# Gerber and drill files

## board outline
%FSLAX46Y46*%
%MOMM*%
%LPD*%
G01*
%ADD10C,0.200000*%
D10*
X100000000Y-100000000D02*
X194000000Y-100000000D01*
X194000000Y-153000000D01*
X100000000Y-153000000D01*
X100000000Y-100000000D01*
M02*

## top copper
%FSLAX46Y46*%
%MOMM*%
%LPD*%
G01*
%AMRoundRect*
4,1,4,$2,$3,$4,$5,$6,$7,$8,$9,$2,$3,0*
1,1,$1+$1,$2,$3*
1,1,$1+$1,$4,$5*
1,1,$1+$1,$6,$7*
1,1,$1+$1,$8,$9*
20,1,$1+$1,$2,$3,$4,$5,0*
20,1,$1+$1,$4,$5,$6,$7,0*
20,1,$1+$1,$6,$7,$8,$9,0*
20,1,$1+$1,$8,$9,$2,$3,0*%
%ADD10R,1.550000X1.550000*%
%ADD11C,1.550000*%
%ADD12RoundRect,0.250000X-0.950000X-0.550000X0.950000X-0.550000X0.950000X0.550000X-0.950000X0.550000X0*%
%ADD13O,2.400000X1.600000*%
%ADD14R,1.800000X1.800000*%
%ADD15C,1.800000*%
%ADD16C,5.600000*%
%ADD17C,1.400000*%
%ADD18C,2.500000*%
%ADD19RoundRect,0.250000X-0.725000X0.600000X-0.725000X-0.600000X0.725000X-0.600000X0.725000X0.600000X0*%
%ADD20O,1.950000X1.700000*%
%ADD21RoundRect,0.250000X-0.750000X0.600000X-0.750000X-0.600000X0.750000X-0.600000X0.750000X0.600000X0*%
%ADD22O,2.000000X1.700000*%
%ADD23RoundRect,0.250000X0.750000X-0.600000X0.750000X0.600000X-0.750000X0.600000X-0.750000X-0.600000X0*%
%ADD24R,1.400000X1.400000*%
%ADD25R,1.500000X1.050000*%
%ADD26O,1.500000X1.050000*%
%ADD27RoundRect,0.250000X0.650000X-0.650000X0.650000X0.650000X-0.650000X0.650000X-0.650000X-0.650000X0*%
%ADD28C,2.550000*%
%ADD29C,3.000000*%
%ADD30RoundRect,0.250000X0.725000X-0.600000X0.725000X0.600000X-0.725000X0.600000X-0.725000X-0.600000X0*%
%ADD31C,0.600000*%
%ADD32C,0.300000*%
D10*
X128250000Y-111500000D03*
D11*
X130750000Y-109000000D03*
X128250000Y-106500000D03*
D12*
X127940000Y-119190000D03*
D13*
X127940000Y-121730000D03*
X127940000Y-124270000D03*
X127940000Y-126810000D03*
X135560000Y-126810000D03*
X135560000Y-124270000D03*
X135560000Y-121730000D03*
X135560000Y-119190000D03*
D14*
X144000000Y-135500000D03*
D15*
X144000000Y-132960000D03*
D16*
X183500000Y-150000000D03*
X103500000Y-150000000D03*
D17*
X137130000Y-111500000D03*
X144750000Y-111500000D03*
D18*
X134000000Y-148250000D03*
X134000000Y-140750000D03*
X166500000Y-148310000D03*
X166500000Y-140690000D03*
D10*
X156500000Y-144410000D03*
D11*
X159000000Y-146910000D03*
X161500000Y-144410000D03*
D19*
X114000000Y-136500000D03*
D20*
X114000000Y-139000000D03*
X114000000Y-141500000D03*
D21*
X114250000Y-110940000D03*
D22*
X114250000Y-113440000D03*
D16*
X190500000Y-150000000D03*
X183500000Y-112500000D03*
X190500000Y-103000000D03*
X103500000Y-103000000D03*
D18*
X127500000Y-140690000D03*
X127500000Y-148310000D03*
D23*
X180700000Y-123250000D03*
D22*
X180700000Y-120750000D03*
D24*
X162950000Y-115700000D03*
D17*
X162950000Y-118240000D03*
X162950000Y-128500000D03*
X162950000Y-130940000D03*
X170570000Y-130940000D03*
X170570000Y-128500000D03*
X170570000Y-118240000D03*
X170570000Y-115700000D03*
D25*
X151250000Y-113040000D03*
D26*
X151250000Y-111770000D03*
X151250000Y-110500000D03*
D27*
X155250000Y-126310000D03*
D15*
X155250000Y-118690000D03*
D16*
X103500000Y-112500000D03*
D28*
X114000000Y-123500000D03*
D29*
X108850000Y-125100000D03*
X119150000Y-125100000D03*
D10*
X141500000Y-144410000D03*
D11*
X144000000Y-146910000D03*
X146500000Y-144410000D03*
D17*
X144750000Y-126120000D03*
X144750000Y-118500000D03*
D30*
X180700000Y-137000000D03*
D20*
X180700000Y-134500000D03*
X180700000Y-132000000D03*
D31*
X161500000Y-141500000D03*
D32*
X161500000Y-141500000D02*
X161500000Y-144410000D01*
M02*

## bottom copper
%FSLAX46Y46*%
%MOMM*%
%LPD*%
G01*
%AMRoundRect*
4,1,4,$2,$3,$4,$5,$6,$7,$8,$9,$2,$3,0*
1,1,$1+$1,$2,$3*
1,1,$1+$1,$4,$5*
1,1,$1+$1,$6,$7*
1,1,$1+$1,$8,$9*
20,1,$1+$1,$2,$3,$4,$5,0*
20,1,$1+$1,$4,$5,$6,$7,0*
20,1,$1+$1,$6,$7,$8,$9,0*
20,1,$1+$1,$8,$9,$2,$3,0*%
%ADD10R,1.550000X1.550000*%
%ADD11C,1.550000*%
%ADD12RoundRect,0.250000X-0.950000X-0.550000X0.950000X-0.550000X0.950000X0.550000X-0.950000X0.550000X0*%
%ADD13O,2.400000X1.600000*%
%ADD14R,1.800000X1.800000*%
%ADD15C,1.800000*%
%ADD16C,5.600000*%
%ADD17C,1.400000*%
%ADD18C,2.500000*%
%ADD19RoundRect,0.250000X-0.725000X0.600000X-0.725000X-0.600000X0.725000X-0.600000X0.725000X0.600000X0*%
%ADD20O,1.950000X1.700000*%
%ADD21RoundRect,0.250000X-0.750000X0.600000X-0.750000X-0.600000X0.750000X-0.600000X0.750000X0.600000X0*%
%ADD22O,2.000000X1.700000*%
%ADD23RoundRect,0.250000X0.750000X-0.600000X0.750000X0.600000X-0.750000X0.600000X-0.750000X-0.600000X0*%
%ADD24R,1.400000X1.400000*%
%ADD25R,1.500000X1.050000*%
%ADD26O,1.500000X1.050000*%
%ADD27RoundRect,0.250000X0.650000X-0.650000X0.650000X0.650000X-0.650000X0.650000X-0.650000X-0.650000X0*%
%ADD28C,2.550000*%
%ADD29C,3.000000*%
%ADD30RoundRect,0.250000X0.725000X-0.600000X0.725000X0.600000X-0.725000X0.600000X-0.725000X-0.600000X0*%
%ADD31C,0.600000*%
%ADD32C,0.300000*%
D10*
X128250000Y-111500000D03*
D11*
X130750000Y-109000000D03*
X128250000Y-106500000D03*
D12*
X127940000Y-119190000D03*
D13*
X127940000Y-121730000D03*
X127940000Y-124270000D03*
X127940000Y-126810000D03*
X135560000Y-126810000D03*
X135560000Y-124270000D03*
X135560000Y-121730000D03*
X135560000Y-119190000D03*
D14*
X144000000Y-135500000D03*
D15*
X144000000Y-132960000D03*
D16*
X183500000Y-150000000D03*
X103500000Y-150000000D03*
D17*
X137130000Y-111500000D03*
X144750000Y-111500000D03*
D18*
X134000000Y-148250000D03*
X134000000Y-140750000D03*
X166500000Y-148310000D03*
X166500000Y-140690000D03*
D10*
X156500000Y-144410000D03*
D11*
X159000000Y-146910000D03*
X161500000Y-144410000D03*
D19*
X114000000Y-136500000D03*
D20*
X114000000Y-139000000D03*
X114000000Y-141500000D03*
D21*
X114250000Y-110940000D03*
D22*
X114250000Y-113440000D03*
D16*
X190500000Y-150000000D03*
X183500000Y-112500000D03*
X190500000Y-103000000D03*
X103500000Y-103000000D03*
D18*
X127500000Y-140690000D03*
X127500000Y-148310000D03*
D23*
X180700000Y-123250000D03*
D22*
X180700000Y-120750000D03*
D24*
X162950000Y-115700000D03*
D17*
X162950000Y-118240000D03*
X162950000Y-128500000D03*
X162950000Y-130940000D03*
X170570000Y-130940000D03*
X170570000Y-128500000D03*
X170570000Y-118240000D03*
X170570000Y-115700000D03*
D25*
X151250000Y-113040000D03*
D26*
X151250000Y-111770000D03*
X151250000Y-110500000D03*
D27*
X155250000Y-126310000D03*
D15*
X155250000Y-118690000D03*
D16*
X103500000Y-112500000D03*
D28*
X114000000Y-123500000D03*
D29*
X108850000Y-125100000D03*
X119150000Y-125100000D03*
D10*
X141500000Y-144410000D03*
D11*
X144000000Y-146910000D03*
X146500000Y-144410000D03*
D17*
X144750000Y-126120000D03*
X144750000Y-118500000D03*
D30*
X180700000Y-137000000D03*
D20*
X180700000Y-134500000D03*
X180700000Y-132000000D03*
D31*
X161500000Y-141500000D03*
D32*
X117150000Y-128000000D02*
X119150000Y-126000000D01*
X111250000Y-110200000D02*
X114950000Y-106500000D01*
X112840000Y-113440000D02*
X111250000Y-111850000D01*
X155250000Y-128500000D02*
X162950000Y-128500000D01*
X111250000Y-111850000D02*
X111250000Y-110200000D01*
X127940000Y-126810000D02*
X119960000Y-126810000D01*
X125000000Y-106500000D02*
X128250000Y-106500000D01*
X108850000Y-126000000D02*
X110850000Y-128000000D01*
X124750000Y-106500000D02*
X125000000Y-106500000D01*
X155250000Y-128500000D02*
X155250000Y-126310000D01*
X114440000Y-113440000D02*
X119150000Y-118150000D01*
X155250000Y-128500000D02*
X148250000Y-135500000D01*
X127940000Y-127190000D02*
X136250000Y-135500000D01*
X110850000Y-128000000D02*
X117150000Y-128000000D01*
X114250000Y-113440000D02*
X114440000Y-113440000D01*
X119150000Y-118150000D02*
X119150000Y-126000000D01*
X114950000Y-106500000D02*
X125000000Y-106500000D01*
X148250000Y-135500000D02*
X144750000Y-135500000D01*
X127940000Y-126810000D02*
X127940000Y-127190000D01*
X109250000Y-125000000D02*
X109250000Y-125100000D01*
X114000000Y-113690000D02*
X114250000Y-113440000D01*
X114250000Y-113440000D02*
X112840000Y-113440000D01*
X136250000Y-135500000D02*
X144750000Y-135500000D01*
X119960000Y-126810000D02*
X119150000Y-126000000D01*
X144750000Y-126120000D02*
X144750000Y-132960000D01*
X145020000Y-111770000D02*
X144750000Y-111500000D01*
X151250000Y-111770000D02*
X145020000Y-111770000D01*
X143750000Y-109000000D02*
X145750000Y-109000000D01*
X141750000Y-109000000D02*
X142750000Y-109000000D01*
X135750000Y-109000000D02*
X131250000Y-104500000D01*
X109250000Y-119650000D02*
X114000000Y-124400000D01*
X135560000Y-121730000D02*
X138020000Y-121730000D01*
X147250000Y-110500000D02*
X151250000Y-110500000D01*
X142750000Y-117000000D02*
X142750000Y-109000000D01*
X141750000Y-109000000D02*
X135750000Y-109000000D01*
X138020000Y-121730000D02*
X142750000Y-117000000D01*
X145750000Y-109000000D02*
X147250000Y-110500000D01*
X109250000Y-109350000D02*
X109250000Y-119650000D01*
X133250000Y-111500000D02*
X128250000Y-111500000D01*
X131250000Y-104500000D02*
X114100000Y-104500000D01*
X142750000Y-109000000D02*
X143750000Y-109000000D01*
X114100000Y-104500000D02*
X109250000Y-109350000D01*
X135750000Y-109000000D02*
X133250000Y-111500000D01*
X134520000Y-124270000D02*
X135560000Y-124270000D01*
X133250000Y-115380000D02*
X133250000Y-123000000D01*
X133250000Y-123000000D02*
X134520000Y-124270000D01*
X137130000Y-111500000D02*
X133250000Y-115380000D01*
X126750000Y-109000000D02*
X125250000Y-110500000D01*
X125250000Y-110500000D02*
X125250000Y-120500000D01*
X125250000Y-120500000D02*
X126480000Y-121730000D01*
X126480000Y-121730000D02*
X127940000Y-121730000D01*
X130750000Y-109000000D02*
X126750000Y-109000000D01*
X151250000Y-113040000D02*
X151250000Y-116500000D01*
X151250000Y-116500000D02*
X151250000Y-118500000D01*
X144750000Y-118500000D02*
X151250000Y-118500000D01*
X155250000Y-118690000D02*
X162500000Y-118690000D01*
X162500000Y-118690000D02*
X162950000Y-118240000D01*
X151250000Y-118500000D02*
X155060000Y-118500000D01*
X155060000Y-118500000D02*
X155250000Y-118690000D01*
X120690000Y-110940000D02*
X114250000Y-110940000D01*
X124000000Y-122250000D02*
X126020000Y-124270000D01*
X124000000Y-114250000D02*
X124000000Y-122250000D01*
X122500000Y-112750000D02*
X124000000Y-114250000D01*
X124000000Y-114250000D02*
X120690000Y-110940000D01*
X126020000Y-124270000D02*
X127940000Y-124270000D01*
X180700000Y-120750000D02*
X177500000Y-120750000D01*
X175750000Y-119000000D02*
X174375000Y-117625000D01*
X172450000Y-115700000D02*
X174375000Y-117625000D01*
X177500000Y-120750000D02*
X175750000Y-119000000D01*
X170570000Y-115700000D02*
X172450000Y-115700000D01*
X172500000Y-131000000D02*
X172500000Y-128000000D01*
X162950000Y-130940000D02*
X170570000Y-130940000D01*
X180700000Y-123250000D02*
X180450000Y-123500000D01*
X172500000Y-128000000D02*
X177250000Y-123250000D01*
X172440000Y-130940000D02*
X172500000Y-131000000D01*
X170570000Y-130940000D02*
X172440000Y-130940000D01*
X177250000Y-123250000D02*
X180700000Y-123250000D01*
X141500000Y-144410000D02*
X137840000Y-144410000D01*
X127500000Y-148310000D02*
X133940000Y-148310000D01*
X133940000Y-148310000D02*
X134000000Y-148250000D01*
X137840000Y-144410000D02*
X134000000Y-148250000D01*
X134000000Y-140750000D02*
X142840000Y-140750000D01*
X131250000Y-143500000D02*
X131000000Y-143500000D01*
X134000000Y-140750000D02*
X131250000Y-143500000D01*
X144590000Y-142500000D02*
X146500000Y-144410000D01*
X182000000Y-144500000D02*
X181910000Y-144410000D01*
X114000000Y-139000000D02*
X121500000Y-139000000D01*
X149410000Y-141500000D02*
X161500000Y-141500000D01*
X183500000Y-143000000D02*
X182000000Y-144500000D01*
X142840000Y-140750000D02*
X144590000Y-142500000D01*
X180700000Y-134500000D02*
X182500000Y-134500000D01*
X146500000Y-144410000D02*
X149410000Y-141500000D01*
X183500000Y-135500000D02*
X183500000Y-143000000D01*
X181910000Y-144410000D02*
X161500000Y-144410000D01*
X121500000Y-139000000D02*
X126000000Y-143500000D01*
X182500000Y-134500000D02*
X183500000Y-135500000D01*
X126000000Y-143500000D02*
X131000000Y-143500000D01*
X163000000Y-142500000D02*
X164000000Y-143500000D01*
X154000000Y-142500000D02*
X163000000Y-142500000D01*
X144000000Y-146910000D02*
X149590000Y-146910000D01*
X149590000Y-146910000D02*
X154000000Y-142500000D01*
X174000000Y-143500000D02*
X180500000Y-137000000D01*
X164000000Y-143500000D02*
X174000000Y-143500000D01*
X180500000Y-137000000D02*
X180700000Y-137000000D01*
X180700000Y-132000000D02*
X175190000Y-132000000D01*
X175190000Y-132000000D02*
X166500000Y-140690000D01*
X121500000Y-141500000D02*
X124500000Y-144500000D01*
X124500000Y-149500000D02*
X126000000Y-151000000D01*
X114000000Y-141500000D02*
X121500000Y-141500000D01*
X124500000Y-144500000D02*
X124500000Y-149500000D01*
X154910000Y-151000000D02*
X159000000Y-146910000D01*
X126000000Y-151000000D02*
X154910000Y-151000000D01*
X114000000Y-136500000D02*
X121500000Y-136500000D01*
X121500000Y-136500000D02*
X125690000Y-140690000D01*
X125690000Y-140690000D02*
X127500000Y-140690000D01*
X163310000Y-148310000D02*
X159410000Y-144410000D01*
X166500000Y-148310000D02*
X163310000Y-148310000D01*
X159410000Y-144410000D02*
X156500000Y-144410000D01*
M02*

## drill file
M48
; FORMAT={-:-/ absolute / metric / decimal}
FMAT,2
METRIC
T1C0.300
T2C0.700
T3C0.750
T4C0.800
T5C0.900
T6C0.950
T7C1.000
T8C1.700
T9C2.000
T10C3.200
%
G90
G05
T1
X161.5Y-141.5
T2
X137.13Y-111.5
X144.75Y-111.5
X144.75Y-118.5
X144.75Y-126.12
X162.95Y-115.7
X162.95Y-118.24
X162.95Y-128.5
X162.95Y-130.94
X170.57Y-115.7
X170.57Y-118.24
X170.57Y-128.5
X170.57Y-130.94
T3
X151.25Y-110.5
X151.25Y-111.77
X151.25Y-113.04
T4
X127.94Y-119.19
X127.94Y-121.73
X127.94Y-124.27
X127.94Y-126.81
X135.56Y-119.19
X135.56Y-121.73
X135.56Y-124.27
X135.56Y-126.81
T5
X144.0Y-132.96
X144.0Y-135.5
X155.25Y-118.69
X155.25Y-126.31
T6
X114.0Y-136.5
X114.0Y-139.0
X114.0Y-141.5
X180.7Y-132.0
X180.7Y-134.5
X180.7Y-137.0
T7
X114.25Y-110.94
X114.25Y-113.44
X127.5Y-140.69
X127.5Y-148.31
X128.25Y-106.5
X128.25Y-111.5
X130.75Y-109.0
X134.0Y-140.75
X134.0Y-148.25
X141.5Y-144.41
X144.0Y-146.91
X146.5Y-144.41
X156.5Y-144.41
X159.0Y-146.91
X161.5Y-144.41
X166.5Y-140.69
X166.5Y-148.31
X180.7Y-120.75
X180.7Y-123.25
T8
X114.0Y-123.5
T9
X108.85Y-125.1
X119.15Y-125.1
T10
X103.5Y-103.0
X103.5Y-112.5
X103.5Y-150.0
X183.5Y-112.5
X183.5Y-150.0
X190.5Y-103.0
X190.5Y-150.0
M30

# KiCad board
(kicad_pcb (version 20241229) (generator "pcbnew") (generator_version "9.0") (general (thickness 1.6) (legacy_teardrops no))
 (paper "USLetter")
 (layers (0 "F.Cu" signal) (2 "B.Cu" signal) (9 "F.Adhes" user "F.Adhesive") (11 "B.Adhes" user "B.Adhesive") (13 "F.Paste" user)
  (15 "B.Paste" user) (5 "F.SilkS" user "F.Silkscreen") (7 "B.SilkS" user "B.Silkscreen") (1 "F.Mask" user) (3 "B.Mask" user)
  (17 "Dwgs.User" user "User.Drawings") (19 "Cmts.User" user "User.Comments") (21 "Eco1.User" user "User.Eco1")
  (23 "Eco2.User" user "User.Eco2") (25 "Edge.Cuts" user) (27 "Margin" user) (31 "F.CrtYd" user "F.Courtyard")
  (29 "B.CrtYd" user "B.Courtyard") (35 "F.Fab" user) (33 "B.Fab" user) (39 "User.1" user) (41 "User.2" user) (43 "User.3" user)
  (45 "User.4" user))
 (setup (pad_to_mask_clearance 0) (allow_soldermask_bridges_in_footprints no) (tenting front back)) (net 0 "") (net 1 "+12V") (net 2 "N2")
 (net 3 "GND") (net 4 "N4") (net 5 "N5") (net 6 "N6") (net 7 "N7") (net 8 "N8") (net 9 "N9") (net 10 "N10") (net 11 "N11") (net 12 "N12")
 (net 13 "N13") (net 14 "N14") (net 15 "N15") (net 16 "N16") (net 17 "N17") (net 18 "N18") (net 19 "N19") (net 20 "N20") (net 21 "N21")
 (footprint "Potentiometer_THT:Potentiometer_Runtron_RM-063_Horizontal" (layer "F.Cu") (at 128.25 111.5 90)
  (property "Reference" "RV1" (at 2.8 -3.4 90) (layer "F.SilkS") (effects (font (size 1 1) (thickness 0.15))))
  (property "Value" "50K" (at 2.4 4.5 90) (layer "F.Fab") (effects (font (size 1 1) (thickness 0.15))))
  (pad "1" thru_hole rect (at 0 0 90) (size 1.55 1.55) (drill 1) (layers "*.Cu" "*.Mask") (remove_unused_layers no) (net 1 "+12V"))
  (pad "2" thru_hole circle (at 2.5 2.5 90) (size 1.55 1.55) (drill 1) (layers "*.Cu" "*.Mask") (remove_unused_layers no) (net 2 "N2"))
  (pad "3" thru_hole circle (at 5 0 90) (size 1.55 1.55) (drill 1) (layers "*.Cu" "*.Mask") (remove_unused_layers no) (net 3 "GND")))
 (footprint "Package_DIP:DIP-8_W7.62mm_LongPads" (layer "F.Cu") (at 127.94 119.19)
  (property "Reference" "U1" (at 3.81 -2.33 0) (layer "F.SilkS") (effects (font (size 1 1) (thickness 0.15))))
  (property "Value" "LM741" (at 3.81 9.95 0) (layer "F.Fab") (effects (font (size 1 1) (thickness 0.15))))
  (pad "1" thru_hole roundrect (at 0 0) (size 2.4 1.6) (drill 0.8) (layers "*.Cu" "*.Mask") (remove_unused_layers no)
   (roundrect_rratio 0.15625) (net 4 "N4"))
  (pad "2" thru_hole oval (at 0 2.54) (size 2.4 1.6) (drill 0.8) (layers "*.Cu" "*.Mask") (remove_unused_layers no) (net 2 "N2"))
  (pad "3" thru_hole oval (at 0 5.08) (size 2.4 1.6) (drill 0.8) (layers "*.Cu" "*.Mask") (remove_unused_layers no) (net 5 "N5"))
  (pad "4" thru_hole oval (at 0 7.62) (size 2.4 1.6) (drill 0.8) (layers "*.Cu" "*.Mask") (remove_unused_layers no) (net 3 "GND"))
  (pad "5" thru_hole oval (at 7.62 7.62) (size 2.4 1.6) (drill 0.8) (layers "*.Cu" "*.Mask") (remove_unused_layers no) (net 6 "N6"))
  (pad "6" thru_hole oval (at 7.62 5.08) (size 2.4 1.6) (drill 0.8) (layers "*.Cu" "*.Mask") (remove_unused_layers no) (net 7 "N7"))
  (pad "7" thru_hole oval (at 7.62 2.54) (size 2.4 1.6) (drill 0.8) (layers "*.Cu" "*.Mask") (remove_unused_layers no) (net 1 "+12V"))
  (pad "8" thru_hole oval (at 7.62 0) (size 2.4 1.6) (drill 0.8) (layers "*.Cu" "*.Mask") (remove_unused_layers no) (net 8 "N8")))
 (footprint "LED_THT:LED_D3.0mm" (layer "F.Cu") (at 144 135.5 90)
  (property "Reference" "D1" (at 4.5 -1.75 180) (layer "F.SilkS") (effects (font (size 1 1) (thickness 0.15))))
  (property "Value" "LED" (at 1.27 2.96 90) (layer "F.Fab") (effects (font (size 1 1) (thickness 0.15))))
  (pad "1" thru_hole rect (at 0 0 90) (size 1.8 1.8) (drill 0.9) (layers "*.Cu" "*.Mask") (remove_unused_layers no) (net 3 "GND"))
  (pad "2" thru_hole circle (at 2.54 0 90) (size 1.8 1.8) (drill 0.9) (layers "*.Cu" "*.Mask") (remove_unused_layers no) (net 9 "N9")))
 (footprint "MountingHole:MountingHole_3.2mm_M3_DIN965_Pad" (layer "F.Cu") (at 183.5 150)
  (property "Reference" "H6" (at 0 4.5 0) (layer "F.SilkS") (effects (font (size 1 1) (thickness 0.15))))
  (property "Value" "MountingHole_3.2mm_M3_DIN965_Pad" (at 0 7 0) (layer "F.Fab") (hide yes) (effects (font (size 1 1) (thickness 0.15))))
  (pad "1" thru_hole circle (at 0 0) (size 5.6 5.6) (drill 3.2) (layers "*.Cu" "*.Mask") (remove_unused_layers no) (zone_connect 2)))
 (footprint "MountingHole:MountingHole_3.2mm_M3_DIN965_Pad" (layer "F.Cu") (at 103.5 150)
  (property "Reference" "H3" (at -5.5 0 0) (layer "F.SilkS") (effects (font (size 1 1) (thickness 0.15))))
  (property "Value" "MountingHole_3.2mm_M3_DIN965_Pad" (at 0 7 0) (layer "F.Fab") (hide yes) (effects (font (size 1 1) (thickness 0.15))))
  (pad "1" thru_hole circle (at 0 0) (size 5.6 5.6) (drill 3.2) (layers "*.Cu" "*.Mask") (remove_unused_layers no) (zone_connect 2)))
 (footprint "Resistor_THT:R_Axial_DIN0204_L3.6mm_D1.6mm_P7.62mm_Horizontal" (layer "F.Cu") (at 137.13 111.5)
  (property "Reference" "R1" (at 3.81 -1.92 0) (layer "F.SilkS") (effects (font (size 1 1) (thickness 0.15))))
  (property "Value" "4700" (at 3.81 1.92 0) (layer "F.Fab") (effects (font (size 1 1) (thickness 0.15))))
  (pad "1" thru_hole circle (at 0 0) (size 1.4 1.4) (drill 0.7) (layers "*.Cu" "*.Mask") (remove_unused_layers no) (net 7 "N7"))
  (pad "2" thru_hole circle (at 7.62 0) (size 1.4 1.4) (drill 0.7) (layers "*.Cu" "*.Mask") (remove_unused_layers no) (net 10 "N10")))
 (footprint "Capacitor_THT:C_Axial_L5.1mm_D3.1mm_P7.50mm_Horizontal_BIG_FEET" (layer "F.Cu") (at 134 148.25 90)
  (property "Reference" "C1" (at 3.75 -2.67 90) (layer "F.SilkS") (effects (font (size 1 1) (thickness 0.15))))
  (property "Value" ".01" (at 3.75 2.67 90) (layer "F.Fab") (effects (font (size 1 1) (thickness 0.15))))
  (pad "1" thru_hole circle (at 0 0 90) (size 2.5 2.5) (drill 1) (layers "*.Cu" "*.Mask") (remove_unused_layers no) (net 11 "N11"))
  (pad "2" thru_hole circle (at 7.5 0 90) (size 2.5 2.5) (drill 1) (layers "*.Cu" "*.Mask") (remove_unused_layers no) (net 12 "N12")))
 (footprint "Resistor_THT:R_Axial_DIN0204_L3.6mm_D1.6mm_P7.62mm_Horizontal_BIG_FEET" (layer "F.Cu") (at 166.5 148.31 90)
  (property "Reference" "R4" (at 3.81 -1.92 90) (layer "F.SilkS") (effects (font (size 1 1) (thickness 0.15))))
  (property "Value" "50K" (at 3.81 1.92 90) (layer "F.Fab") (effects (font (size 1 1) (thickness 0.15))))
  (pad "1" thru_hole circle (at 0 0 90) (size 2.5 2.5) (drill 1) (layers "*.Cu" "*.Mask") (remove_unused_layers no) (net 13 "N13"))
  (pad "2" thru_hole circle (at 7.62 0 90) (size 2.5 2.5) (drill 1) (layers "*.Cu" "*.Mask") (remove_unused_layers no) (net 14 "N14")))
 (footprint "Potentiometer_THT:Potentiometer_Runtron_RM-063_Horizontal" (layer "F.Cu") (at 156.5 144.41)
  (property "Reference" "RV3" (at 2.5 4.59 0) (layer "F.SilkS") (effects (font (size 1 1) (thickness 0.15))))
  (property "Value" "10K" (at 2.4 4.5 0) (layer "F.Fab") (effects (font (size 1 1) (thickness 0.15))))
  (pad "1" thru_hole rect (at 0 0) (size 1.55 1.55) (drill 1) (layers "*.Cu" "*.Mask") (remove_unused_layers no) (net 13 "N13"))
  (pad "2" thru_hole circle (at 2.5 2.5) (size 1.55 1.55) (drill 1) (layers "*.Cu" "*.Mask") (remove_unused_layers no) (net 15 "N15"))
  (pad "3" thru_hole circle (at 5 0) (size 1.55 1.55) (drill 1) (layers "*.Cu" "*.Mask") (remove_unused_layers no) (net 12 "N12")))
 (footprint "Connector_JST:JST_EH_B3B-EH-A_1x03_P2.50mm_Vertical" (layer "F.Cu") (at 114 136.5 -90)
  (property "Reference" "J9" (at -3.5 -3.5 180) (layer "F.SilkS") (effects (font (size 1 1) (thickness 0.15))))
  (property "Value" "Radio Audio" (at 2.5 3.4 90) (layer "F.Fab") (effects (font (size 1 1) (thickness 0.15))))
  (pad "1" thru_hole roundrect (at 0 0 270) (size 1.7 1.95) (drill 0.95) (layers "*.Cu" "*.Mask") (remove_unused_layers no)
   (roundrect_rratio 0.147059) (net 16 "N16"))
  (pad "2" thru_hole oval (at 2.5 0 270) (size 1.7 1.95) (drill 0.95) (layers "*.Cu" "*.Mask") (remove_unused_layers no) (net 12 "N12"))
  (pad "3" thru_hole oval (at 5 0 270) (size 1.7 1.95) (drill 0.95) (layers "*.Cu" "*.Mask") (remove_unused_layers no) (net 15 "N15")))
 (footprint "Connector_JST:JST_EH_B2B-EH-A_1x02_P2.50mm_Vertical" (layer "F.Cu") (at 114.25 110.94 -90)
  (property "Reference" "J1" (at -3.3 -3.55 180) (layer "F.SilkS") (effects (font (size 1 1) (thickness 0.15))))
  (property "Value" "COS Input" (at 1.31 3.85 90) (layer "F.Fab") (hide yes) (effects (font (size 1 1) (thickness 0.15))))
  (pad "1" thru_hole roundrect (at 0 0 270) (size 1.7 2) (drill 1) (layers "*.Cu" "*.Mask") (remove_unused_layers no)
   (roundrect_rratio 0.147059) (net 5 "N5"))
  (pad "2" thru_hole oval (at 2.5 0 270) (size 1.7 2) (drill 1) (layers "*.Cu" "*.Mask") (remove_unused_layers no) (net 3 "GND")))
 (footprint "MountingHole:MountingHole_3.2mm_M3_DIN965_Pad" (layer "F.Cu") (at 190.5 150)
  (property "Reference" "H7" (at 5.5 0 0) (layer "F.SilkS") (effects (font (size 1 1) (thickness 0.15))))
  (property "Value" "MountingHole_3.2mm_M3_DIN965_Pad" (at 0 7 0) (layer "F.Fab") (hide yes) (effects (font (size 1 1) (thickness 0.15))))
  (pad "1" thru_hole circle (at 0 0) (size 5.6 5.6) (drill 3.2) (layers "*.Cu" "*.Mask") (remove_unused_layers no) (zone_connect 2)))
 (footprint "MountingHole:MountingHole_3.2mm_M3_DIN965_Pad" (layer "F.Cu") (at 183.5 112.5)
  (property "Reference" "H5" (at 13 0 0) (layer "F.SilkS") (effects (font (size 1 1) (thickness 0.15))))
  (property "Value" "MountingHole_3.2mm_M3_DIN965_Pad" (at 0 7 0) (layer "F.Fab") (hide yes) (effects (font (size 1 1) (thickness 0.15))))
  (pad "1" thru_hole circle (at 0 0) (size 5.6 5.6) (drill 3.2) (layers "*.Cu" "*.Mask") (remove_unused_layers no) (zone_connect 2)))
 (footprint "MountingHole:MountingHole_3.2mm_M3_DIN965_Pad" (layer "F.Cu") (at 190.5 103)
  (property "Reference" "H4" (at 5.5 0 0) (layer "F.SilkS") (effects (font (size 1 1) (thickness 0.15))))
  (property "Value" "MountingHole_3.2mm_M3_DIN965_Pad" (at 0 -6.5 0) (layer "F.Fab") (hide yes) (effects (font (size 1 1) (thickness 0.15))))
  (pad "1" thru_hole circle (at 0 0) (size 5.6 5.6) (drill 3.2) (layers "*.Cu" "*.Mask") (remove_unused_layers no) (zone_connect 2)))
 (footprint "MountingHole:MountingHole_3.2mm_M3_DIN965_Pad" (layer "F.Cu") (at 103.5 103)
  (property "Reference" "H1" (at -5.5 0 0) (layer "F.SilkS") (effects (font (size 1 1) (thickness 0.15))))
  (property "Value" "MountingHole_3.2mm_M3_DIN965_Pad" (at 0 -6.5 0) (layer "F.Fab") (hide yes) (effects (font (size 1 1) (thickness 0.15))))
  (pad "1" thru_hole circle (at 0 0) (size 5.6 5.6) (drill 3.2) (layers "*.Cu" "*.Mask") (remove_unused_layers no) (zone_connect 2)))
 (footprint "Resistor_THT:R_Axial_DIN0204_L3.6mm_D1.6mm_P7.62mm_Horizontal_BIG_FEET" (layer "F.Cu") (at 127.5 140.69 -90)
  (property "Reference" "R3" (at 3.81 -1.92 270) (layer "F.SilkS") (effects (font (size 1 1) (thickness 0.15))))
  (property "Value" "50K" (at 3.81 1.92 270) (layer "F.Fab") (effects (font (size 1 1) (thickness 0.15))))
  (pad "1" thru_hole circle (at 0 0 270) (size 2.5 2.5) (drill 1) (layers "*.Cu" "*.Mask") (remove_unused_layers no) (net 16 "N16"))
  (pad "2" thru_hole circle (at 7.62 0 270) (size 2.5 2.5) (drill 1) (layers "*.Cu" "*.Mask") (remove_unused_layers no) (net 11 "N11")))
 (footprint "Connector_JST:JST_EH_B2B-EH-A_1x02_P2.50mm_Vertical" (layer "F.Cu") (at 180.7 123.25 90)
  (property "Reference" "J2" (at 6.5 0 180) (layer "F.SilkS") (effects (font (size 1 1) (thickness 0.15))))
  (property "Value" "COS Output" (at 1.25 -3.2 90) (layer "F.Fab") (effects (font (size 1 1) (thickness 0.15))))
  (pad "1" thru_hole roundrect (at 0 0 90) (size 1.7 2) (drill 1) (layers "*.Cu" "*.Mask") (remove_unused_layers no)
   (roundrect_rratio 0.147059) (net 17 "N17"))
  (pad "2" thru_hole oval (at 2.5 0 90) (size 1.7 2) (drill 1) (layers "*.Cu" "*.Mask") (remove_unused_layers no) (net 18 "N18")))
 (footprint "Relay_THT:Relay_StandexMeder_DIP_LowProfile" (layer "F.Cu") (at 162.95 115.7)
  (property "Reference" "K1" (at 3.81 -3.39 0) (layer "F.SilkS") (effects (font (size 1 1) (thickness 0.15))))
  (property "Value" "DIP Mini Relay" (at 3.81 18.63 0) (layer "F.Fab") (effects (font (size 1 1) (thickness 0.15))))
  (pad "1" thru_hole rect (at 0 0) (size 1.4 1.4) (drill 0.7) (layers "*.Cu" "*.Mask") (remove_unused_layers no) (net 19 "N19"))
  (pad "2" thru_hole circle (at 0 2.54) (size 1.4 1.4) (drill 0.7) (layers "*.Cu" "*.Mask") (remove_unused_layers no) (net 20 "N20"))
  (pad "6" thru_hole circle (at 0 12.8) (size 1.4 1.4) (drill 0.7) (layers "*.Cu" "*.Mask") (remove_unused_layers no) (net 3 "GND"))
  (pad "7" thru_hole circle (at 0 15.24) (size 1.4 1.4) (drill 0.7) (layers "*.Cu" "*.Mask") (remove_unused_layers no) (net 17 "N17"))
  (pad "8" thru_hole circle (at 7.62 15.24) (size 1.4 1.4) (drill 0.7) (layers "*.Cu" "*.Mask") (remove_unused_layers no) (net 17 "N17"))
  (pad "9" thru_hole circle (at 7.62 12.8) (size 1.4 1.4) (drill 0.7) (layers "*.Cu" "*.Mask") (remove_unused_layers no))
  (pad "13" thru_hole circle (at 7.62 2.54) (size 1.4 1.4) (drill 0.7) (layers "*.Cu" "*.Mask") (remove_unused_layers no))
  (pad "14" thru_hole circle (at 7.62 0) (size 1.4 1.4) (drill 0.7) (layers "*.Cu" "*.Mask") (remove_unused_layers no) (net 18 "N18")))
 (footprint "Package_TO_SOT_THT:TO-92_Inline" (layer "F.Cu") (at 151.25 113.04 90)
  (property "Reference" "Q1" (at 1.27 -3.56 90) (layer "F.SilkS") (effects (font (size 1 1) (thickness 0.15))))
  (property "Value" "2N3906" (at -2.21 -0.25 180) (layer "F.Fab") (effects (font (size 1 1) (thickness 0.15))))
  (pad "1" thru_hole rect (at 0 0 90) (size 1.05 1.5) (drill 0.75) (layers "*.Cu" "*.Mask") (remove_unused_layers no) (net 20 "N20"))
  (pad "2" thru_hole oval (at 1.27 0 90) (size 1.05 1.5) (drill 0.75) (layers "*.Cu" "*.Mask") (remove_unused_layers no) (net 10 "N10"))
  (pad "3" thru_hole oval (at 2.54 0 90) (size 1.05 1.5) (drill 0.75) (layers "*.Cu" "*.Mask") (remove_unused_layers no) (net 1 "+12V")))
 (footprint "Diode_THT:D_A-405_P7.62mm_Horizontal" (layer "F.Cu") (at 155.25 126.31 90)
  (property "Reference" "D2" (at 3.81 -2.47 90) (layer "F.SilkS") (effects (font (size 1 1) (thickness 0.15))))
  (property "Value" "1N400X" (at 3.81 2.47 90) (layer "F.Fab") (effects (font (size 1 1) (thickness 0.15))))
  (pad "1" thru_hole roundrect (at 0 0 90) (size 1.8 1.8) (drill 0.9) (layers "*.Cu" "*.Mask") (remove_unused_layers no)
   (roundrect_rratio 0.138889) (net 3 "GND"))
  (pad "2" thru_hole circle (at 7.62 0 90) (size 1.8 1.8) (drill 0.9) (layers "*.Cu" "*.Mask") (remove_unused_layers no) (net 20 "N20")))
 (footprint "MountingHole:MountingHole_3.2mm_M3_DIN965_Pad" (layer "F.Cu") (at 103.5 112.5)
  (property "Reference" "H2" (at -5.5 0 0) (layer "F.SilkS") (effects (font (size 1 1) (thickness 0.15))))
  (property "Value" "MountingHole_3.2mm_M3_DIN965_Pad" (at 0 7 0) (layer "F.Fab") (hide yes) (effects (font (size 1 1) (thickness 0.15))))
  (pad "1" thru_hole circle (at 0 0) (size 5.6 5.6) (drill 3.2) (layers "*.Cu" "*.Mask") (remove_unused_layers no) (zone_connect 2)))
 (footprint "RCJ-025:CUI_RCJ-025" (layer "F.Cu") (at 114 125.1)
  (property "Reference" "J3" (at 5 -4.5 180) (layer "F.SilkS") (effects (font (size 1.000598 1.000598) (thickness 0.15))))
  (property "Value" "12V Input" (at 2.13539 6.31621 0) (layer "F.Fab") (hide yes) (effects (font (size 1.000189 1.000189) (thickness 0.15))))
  (pad "1" thru_hole circle (at 0 -1.6) (size 2.55 2.55) (drill 1.7) (layers "*.Cu" "*.Mask") (remove_unused_layers no) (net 1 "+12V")
   (solder_mask_margin 0.102))
  (pad "2" thru_hole circle (at -5.15 0) (size 3 3) (drill 2) (layers "*.Cu" "*.Mask") (remove_unused_layers no) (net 3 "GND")
   (solder_mask_margin 0.102))
  (pad "2" thru_hole circle (at 5.15 0) (size 3 3) (drill 2) (layers "*.Cu" "*.Mask") (remove_unused_layers no) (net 3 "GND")
   (solder_mask_margin 0.102)))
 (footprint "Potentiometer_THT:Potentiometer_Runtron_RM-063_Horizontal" (layer "F.Cu") (at 141.5 144.41)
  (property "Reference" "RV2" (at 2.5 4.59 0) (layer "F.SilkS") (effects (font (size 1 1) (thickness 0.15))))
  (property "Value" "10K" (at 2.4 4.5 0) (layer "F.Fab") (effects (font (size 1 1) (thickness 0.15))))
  (pad "1" thru_hole rect (at 0 0) (size 1.55 1.55) (drill 1) (layers "*.Cu" "*.Mask") (remove_unused_layers no) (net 11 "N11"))
  (pad "2" thru_hole circle (at 2.5 2.5) (size 1.55 1.55) (drill 1) (layers "*.Cu" "*.Mask") (remove_unused_layers no) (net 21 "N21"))
  (pad "3" thru_hole circle (at 5 0) (size 1.55 1.55) (drill 1) (layers "*.Cu" "*.Mask") (remove_unused_layers no) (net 12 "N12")))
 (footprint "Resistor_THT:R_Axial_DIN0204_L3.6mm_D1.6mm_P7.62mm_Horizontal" (layer "F.Cu") (at 144.75 126.12 90)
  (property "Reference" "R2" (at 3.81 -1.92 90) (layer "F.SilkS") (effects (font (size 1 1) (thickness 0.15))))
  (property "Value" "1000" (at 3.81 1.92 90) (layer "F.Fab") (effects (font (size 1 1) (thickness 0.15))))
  (pad "1" thru_hole circle (at 0 0 90) (size 1.4 1.4) (drill 0.7) (layers "*.Cu" "*.Mask") (remove_unused_layers no) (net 9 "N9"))
  (pad "2" thru_hole circle (at 7.62 0 90) (size 1.4 1.4) (drill 0.7) (layers "*.Cu" "*.Mask") (remove_unused_layers no) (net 20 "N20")))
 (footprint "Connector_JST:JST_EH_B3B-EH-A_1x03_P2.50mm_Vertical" (layer "F.Cu") (at 180.7 137 90)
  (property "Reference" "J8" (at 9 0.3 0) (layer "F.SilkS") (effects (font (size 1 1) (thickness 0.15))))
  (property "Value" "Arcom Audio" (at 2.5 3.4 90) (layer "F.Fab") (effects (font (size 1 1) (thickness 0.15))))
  (pad "1" thru_hole roundrect (at 0 0 90) (size 1.7 1.95) (drill 0.95) (layers "*.Cu" "*.Mask") (remove_unused_layers no)
   (roundrect_rratio 0.147059) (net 21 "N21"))
  (pad "2" thru_hole oval (at 2.5 0 90) (size 1.7 1.95) (drill 0.95) (layers "*.Cu" "*.Mask") (remove_unused_layers no) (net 12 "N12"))
  (pad "3" thru_hole oval (at 5 0 90) (size 1.7 1.95) (drill 0.95) (layers "*.Cu" "*.Mask") (remove_unused_layers no) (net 14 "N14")))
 (gr_rect (start 100 100) (end 194 153) (stroke (width 0.2) (type solid)) (fill no) (locked yes) (layer "Edge.Cuts"))
 (segment (start 117.15 128) (end 119.15 126) (width 0.3) (layer "B.Cu") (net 3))
 (segment (start 111.25 110.2) (end 114.95 106.5) (width 0.3) (layer "B.Cu") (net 3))
 (segment (start 112.84 113.44) (end 111.25 111.85) (width 0.3) (layer "B.Cu") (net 3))
 (segment (start 155.25 128.5) (end 162.95 128.5) (width 0.3) (layer "B.Cu") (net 3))
 (segment (start 111.25 111.85) (end 111.25 110.2) (width 0.3) (layer "B.Cu") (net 3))
 (segment (start 127.94 126.81) (end 119.96 126.81) (width 0.3) (layer "B.Cu") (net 3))
 (segment (start 125 106.5) (end 128.25 106.5) (width 0.3) (layer "B.Cu") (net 3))
 (segment (start 108.85 126) (end 110.85 128) (width 0.3) (layer "B.Cu") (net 3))
 (segment (start 124.75 106.5) (end 125 106.5) (width 0.3) (layer "B.Cu") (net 3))
 (segment (start 155.25 128.5) (end 155.25 126.31) (width 0.3) (layer "B.Cu") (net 3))
 (segment (start 114.44 113.44) (end 119.15 118.15) (width 0.3) (layer "B.Cu") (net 3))
 (segment (start 155.25 128.5) (end 148.25 135.5) (width 0.3) (layer "B.Cu") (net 3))
 (segment (start 127.94 127.19) (end 136.25 135.5) (width 0.3) (layer "B.Cu") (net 3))
 (segment (start 110.85 128) (end 117.15 128) (width 0.3) (layer "B.Cu") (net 3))
 (segment (start 114.25 113.44) (end 114.44 113.44) (width 0.3) (layer "B.Cu") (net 3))
 (segment (start 119.15 118.15) (end 119.15 126) (width 0.3) (layer "B.Cu") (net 3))
 (segment (start 114.95 106.5) (end 125 106.5) (width 0.3) (layer "B.Cu") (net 3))
 (segment (start 148.25 135.5) (end 144.75 135.5) (width 0.3) (layer "B.Cu") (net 3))
 (segment (start 127.94 126.81) (end 127.94 127.19) (width 0.3) (layer "B.Cu") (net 3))
 (segment (start 109.25 125) (end 109.25 125.1) (width 0.3) (layer "B.Cu") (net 3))
 (segment (start 114 113.69) (end 114.25 113.44) (width 0.3) (layer "B.Cu") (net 3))
 (segment (start 114.25 113.44) (end 112.84 113.44) (width 0.3) (layer "B.Cu") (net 3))
 (segment (start 136.25 135.5) (end 144.75 135.5) (width 0.3) (layer "B.Cu") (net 3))
 (segment (start 119.96 126.81) (end 119.15 126) (width 0.3) (layer "B.Cu") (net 3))
 (segment (start 144.75 126.12) (end 144.75 132.96) (width 0.3) (layer "B.Cu") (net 9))
 (segment (start 145.02 111.77) (end 144.75 111.5) (width 0.3) (layer "B.Cu") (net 10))
 (segment (start 151.25 111.77) (end 145.02 111.77) (width 0.3) (layer "B.Cu") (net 10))
 (segment (start 143.75 109) (end 145.75 109) (width 0.3) (layer "B.Cu") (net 1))
 (segment (start 141.75 109) (end 142.75 109) (width 0.3) (layer "B.Cu") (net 1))
 (segment (start 135.75 109) (end 131.25 104.5) (width 0.3) (layer "B.Cu") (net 1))
 (segment (start 109.25 119.65) (end 114 124.4) (width 0.3) (layer "B.Cu") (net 1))
 (segment (start 135.56 121.73) (end 138.02 121.73) (width 0.3) (layer "B.Cu") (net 1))
 (segment (start 147.25 110.5) (end 151.25 110.5) (width 0.3) (layer "B.Cu") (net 1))
 (segment (start 142.75 117) (end 142.75 109) (width 0.3) (layer "B.Cu") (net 1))
 (segment (start 141.75 109) (end 135.75 109) (width 0.3) (layer "B.Cu") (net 1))
 (segment (start 138.02 121.73) (end 142.75 117) (width 0.3) (layer "B.Cu") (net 1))
 (segment (start 145.75 109) (end 147.25 110.5) (width 0.3) (layer "B.Cu") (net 1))
 (segment (start 109.25 109.35) (end 109.25 119.65) (width 0.3) (layer "B.Cu") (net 1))
 (segment (start 133.25 111.5) (end 128.25 111.5) (width 0.3) (layer "B.Cu") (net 1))
 (segment (start 131.25 104.5) (end 114.1 104.5) (width 0.3) (layer "B.Cu") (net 1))
 (segment (start 142.75 109) (end 143.75 109) (width 0.3) (layer "B.Cu") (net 1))
 (segment (start 114.1 104.5) (end 109.25 109.35) (width 0.3) (layer "B.Cu") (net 1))
 (segment (start 135.75 109) (end 133.25 111.5) (width 0.3) (layer "B.Cu") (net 1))
 (segment (start 134.52 124.27) (end 135.56 124.27) (width 0.3) (layer "B.Cu") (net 7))
 (segment (start 133.25 115.38) (end 133.25 123) (width 0.3) (layer "B.Cu") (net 7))
 (segment (start 133.25 123) (end 134.52 124.27) (width 0.3) (layer "B.Cu") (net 7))
 (segment (start 137.13 111.5) (end 133.25 115.38) (width 0.3) (layer "B.Cu") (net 7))
 (segment (start 126.75 109) (end 125.25 110.5) (width 0.3) (layer "B.Cu") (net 2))
 (segment (start 125.25 110.5) (end 125.25 120.5) (width 0.3) (layer "B.Cu") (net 2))
 (segment (start 125.25 120.5) (end 126.48 121.73) (width 0.3) (layer "B.Cu") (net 2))
 (segment (start 126.48 121.73) (end 127.94 121.73) (width 0.3) (layer "B.Cu") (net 2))
 (segment (start 130.75 109) (end 126.75 109) (width 0.3) (layer "B.Cu") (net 2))
 (segment (start 151.25 113.04) (end 151.25 116.5) (width 0.3) (layer "B.Cu") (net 20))
 (segment (start 151.25 116.5) (end 151.25 118.5) (width 0.3) (layer "B.Cu") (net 20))
 (segment (start 144.75 118.5) (end 151.25 118.5) (width 0.3) (layer "B.Cu") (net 20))
 (segment (start 155.25 118.69) (end 162.5 118.69) (width 0.3) (layer "B.Cu") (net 20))
 (segment (start 162.5 118.69) (end 162.95 118.24) (width 0.3) (layer "B.Cu") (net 20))
 (segment (start 151.25 118.5) (end 155.06 118.5) (width 0.3) (layer "B.Cu") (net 20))
 (segment (start 155.06 118.5) (end 155.25 118.69) (width 0.3) (layer "B.Cu") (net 20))
 (segment (start 120.69 110.94) (end 114.25 110.94) (width 0.3) (layer "B.Cu") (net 5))
 (segment (start 124 122.25) (end 126.02 124.27) (width 0.3) (layer "B.Cu") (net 5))
 (segment (start 124 114.25) (end 124 122.25) (width 0.3) (layer "B.Cu") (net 5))
 (segment (start 122.5 112.75) (end 124 114.25) (width 0.3) (layer "B.Cu") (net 5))
 (segment (start 124 114.25) (end 120.69 110.94) (width 0.3) (layer "B.Cu") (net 5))
 (segment (start 126.02 124.27) (end 127.94 124.27) (width 0.3) (layer "B.Cu") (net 5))
 (segment (start 180.7 120.75) (end 177.5 120.75) (width 0.3) (layer "B.Cu") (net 18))
 (segment (start 175.75 119) (end 174.375 117.625) (width 0.3) (layer "B.Cu") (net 18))
 (segment (start 172.45 115.7) (end 174.375 117.625) (width 0.3) (layer "B.Cu") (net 18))
 (segment (start 177.5 120.75) (end 175.75 119) (width 0.3) (layer "B.Cu") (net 18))
 (segment (start 170.57 115.7) (end 172.45 115.7) (width 0.3) (layer "B.Cu") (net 18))
 (segment (start 172.5 131) (end 172.5 128) (width 0.3) (layer "B.Cu") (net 17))
 (segment (start 162.95 130.94) (end 170.57 130.94) (width 0.3) (layer "B.Cu") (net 17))
 (segment (start 180.7 123.25) (end 180.45 123.5) (width 0.3) (layer "B.Cu") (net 17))
 (segment (start 172.5 128) (end 177.25 123.25) (width 0.3) (layer "B.Cu") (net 17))
 (segment (start 172.44 130.94) (end 172.5 131) (width 0.3) (layer "B.Cu") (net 17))
 (segment (start 170.57 130.94) (end 172.44 130.94) (width 0.3) (layer "B.Cu") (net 17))
 (segment (start 177.25 123.25) (end 180.7 123.25) (width 0.3) (layer "B.Cu") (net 17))
 (segment (start 141.5 144.41) (end 137.84 144.41) (width 0.3) (layer "B.Cu") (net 11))
 (segment (start 127.5 148.31) (end 133.94 148.31) (width 0.3) (layer "B.Cu") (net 11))
 (segment (start 133.94 148.31) (end 134 148.25) (width 0.3) (layer "B.Cu") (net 11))
 (segment (start 137.84 144.41) (end 134 148.25) (width 0.3) (layer "B.Cu") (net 11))
 (segment (start 161.5 141.5) (end 161.5 144.41) (width 0.3) (layer "F.Cu") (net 12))
 (via (at 161.5 141.5) (size 0.6) (drill 0.3) (layers "F.Cu" "B.Cu") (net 12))
 (segment (start 134 140.75) (end 142.84 140.75) (width 0.3) (layer "B.Cu") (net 12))
 (segment (start 131.25 143.5) (end 131 143.5) (width 0.3) (layer "B.Cu") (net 12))
 (segment (start 134 140.75) (end 131.25 143.5) (width 0.3) (layer "B.Cu") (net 12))
 (segment (start 144.59 142.5) (end 146.5 144.41) (width 0.3) (layer "B.Cu") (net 12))
 (segment (start 182 144.5) (end 181.91 144.41) (width 0.3) (layer "B.Cu") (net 12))
 (segment (start 114 139) (end 121.5 139) (width 0.3) (layer "B.Cu") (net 12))
 (segment (start 149.41 141.5) (end 161.5 141.5) (width 0.3) (layer "B.Cu") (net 12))
 (segment (start 183.5 143) (end 182 144.5) (width 0.3) (layer "B.Cu") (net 12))
 (segment (start 142.84 140.75) (end 144.59 142.5) (width 0.3) (layer "B.Cu") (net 12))
 (segment (start 180.7 134.5) (end 182.5 134.5) (width 0.3) (layer "B.Cu") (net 12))
 (segment (start 146.5 144.41) (end 149.41 141.5) (width 0.3) (layer "B.Cu") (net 12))
 (segment (start 183.5 135.5) (end 183.5 143) (width 0.3) (layer "B.Cu") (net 12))
 (segment (start 181.91 144.41) (end 161.5 144.41) (width 0.3) (layer "B.Cu") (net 12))
 (segment (start 121.5 139) (end 126 143.5) (width 0.3) (layer "B.Cu") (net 12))
 (segment (start 182.5 134.5) (end 183.5 135.5) (width 0.3) (layer "B.Cu") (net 12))
 (segment (start 126 143.5) (end 131 143.5) (width 0.3) (layer "B.Cu") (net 12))
 (segment (start 163 142.5) (end 164 143.5) (width 0.3) (layer "B.Cu") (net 21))
 (segment (start 154 142.5) (end 163 142.5) (width 0.3) (layer "B.Cu") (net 21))
 (segment (start 144 146.91) (end 149.59 146.91) (width 0.3) (layer "B.Cu") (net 21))
 (segment (start 149.59 146.91) (end 154 142.5) (width 0.3) (layer "B.Cu") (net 21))
 (segment (start 174 143.5) (end 180.5 137) (width 0.3) (layer "B.Cu") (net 21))
 (segment (start 164 143.5) (end 174 143.5) (width 0.3) (layer "B.Cu") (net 21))
 (segment (start 180.5 137) (end 180.7 137) (width 0.3) (layer "B.Cu") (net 21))
 (segment (start 180.7 132) (end 175.19 132) (width 0.3) (layer "B.Cu") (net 14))
 (segment (start 175.19 132) (end 166.5 140.69) (width 0.3) (layer "B.Cu") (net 14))
 (segment (start 121.5 141.5) (end 124.5 144.5) (width 0.3) (layer "B.Cu") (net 15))
 (segment (start 124.5 149.5) (end 126 151) (width 0.3) (layer "B.Cu") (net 15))
 (segment (start 114 141.5) (end 121.5 141.5) (width 0.3) (layer "B.Cu") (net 15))
 (segment (start 124.5 144.5) (end 124.5 149.5) (width 0.3) (layer "B.Cu") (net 15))
 (segment (start 154.91 151) (end 159 146.91) (width 0.3) (layer "B.Cu") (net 15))
 (segment (start 126 151) (end 154.91 151) (width 0.3) (layer "B.Cu") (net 15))
 (segment (start 114 136.5) (end 121.5 136.5) (width 0.3) (layer "B.Cu") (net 16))
 (segment (start 121.5 136.5) (end 125.69 140.69) (width 0.3) (layer "B.Cu") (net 16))
 (segment (start 125.69 140.69) (end 127.5 140.69) (width 0.3) (layer "B.Cu") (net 16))
 (segment (start 163.31 148.31) (end 159.41 144.41) (width 0.3) (layer "B.Cu") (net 13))
 (segment (start 166.5 148.31) (end 163.31 148.31) (width 0.3) (layer "B.Cu") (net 13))
 (segment (start 159.41 144.41) (end 156.5 144.41) (width 0.3) (layer "B.Cu") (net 13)))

